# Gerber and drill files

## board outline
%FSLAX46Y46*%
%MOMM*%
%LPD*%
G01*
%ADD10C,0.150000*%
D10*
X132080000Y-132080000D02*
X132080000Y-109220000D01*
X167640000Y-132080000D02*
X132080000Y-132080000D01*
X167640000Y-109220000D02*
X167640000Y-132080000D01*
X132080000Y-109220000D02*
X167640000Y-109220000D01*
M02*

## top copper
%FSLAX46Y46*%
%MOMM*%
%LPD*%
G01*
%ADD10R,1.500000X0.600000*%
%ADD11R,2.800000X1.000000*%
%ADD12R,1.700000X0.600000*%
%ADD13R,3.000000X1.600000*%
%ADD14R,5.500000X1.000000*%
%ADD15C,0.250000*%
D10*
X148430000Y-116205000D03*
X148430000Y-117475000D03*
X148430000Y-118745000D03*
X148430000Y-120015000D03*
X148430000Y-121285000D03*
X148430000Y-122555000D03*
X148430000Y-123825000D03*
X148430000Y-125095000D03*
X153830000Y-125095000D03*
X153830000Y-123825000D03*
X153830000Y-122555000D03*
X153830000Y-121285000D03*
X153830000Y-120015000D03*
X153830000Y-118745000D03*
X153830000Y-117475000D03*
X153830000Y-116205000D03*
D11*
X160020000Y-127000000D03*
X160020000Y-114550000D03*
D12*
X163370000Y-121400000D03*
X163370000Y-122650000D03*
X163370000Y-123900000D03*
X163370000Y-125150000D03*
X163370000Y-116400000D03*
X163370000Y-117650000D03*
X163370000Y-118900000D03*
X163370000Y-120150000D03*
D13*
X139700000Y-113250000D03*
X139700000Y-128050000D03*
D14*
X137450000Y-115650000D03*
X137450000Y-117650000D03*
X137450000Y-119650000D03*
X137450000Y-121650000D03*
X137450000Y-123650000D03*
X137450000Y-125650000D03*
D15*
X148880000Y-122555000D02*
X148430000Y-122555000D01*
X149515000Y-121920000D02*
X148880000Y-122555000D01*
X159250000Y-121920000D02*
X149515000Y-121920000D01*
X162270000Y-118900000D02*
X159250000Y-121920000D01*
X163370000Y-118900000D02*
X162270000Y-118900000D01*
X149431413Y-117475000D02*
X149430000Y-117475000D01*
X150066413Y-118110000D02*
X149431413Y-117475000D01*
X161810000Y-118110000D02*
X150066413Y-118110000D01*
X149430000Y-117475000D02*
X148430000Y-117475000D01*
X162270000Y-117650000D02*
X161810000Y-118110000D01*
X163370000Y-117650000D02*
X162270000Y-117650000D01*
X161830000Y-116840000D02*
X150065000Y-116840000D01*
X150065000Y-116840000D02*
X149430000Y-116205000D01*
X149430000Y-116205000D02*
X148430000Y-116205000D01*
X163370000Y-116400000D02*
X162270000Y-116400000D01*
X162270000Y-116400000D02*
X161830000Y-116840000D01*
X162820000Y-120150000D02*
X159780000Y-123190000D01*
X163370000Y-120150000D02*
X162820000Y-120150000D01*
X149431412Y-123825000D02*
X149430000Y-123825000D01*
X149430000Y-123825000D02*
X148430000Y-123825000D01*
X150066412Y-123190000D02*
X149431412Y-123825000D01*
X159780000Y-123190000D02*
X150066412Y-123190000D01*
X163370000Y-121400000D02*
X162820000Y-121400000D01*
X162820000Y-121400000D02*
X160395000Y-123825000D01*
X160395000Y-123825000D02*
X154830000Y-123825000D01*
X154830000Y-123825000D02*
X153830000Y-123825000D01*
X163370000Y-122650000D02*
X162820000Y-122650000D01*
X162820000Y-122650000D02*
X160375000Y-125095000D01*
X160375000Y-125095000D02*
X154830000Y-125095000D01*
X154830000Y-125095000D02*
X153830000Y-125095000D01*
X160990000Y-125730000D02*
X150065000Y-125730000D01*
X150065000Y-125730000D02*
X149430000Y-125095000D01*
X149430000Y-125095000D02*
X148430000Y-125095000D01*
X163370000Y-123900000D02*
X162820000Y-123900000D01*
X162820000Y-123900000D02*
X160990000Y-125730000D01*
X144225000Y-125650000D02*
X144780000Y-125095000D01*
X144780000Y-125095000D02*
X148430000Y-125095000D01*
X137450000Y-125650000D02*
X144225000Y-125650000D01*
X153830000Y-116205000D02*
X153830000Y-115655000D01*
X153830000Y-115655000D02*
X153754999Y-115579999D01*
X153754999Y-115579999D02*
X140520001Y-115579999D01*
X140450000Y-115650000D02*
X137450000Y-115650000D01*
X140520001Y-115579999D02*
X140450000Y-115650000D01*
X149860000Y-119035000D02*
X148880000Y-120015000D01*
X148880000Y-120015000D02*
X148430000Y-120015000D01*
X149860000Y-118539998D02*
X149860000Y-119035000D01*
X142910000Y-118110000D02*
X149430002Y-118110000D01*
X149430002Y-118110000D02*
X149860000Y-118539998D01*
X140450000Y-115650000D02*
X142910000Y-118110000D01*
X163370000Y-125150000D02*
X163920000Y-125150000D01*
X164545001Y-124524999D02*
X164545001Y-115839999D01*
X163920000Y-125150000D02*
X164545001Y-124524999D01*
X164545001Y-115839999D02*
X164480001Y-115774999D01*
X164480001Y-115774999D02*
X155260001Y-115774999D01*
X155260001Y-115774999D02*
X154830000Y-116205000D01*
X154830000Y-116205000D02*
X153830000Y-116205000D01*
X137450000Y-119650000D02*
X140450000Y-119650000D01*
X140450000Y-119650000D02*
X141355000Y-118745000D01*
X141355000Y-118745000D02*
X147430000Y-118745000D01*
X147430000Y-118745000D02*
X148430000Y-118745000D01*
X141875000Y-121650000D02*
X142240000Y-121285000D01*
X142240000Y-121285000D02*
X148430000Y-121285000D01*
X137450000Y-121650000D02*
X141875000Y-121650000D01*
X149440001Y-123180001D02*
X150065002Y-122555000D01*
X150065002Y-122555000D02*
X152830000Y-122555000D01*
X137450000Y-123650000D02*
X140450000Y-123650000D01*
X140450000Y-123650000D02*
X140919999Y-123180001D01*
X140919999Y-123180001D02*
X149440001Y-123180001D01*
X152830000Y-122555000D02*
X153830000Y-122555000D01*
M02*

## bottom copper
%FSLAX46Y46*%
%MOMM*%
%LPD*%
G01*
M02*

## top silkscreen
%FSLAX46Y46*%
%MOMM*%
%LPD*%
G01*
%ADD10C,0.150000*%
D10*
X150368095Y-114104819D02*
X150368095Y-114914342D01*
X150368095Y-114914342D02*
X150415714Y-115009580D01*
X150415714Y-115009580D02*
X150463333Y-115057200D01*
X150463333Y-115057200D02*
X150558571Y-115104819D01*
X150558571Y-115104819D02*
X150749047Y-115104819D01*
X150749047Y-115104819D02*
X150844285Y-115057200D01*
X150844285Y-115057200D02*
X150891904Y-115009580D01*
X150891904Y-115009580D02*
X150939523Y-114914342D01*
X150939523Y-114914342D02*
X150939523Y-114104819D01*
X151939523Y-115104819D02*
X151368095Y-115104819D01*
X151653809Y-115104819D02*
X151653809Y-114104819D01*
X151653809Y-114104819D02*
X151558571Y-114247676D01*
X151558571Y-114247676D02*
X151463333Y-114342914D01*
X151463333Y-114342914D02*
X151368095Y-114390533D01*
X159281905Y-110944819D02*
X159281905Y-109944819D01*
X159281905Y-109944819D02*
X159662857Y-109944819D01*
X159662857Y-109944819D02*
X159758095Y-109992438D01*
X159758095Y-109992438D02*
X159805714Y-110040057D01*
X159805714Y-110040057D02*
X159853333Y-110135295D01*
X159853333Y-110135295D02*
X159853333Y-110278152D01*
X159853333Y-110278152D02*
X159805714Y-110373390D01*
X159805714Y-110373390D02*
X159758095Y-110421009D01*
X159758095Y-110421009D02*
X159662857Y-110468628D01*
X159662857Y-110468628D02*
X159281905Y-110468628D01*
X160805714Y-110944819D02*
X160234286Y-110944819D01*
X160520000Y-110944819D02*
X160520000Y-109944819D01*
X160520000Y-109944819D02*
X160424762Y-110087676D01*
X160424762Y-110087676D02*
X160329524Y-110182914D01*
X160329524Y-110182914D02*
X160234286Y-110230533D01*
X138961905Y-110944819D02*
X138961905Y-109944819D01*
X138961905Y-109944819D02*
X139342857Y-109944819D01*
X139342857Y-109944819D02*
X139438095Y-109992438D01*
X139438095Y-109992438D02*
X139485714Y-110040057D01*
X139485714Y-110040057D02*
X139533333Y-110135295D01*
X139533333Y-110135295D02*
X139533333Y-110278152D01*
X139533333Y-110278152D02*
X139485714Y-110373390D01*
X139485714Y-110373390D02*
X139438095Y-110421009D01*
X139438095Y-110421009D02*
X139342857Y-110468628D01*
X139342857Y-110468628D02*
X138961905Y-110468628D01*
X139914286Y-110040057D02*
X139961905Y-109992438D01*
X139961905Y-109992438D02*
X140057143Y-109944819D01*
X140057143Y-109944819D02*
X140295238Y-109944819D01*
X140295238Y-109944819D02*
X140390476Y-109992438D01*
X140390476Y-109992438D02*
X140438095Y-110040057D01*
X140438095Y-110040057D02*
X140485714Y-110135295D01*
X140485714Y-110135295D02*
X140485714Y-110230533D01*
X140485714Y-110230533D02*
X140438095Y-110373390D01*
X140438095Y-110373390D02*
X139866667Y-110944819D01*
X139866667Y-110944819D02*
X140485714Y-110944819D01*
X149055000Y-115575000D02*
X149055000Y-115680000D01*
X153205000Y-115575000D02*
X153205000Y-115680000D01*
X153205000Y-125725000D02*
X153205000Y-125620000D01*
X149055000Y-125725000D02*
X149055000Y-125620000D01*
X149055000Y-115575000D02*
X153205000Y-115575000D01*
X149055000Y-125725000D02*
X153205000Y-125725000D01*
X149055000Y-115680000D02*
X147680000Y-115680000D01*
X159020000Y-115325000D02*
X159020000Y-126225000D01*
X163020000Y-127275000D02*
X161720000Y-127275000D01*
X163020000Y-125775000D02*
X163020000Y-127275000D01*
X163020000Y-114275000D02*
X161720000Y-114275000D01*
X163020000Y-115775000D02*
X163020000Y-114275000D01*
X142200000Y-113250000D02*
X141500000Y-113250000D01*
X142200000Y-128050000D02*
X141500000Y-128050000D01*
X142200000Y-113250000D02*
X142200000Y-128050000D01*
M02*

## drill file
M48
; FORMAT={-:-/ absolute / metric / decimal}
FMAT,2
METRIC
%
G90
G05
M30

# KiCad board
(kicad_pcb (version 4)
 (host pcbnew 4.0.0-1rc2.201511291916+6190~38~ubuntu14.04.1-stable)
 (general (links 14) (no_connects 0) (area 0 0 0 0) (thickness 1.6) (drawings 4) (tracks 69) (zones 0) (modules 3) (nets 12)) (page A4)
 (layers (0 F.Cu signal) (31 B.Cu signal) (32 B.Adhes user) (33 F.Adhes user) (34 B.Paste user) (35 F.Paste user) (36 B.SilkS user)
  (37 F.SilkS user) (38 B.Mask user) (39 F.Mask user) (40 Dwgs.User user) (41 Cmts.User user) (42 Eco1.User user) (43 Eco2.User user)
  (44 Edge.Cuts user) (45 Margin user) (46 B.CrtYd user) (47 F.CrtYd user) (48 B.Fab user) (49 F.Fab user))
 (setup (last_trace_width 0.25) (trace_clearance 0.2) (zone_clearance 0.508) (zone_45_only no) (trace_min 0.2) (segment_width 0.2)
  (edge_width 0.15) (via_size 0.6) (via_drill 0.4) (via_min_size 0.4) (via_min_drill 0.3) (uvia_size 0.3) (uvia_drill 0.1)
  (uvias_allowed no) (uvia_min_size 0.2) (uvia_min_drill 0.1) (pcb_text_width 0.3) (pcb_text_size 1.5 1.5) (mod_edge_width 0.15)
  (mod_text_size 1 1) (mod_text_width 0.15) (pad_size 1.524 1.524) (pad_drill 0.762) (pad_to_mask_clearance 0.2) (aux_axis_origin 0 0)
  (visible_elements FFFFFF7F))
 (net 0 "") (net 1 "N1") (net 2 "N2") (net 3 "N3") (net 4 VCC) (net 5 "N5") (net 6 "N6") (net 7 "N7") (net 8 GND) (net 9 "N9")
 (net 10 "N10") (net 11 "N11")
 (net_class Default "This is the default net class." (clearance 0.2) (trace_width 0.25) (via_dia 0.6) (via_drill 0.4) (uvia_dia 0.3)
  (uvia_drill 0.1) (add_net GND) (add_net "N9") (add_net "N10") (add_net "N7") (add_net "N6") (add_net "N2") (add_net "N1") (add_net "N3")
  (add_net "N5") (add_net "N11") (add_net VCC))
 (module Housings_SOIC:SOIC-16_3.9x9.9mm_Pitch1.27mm (layer F.Cu) (at 151.13 120.65)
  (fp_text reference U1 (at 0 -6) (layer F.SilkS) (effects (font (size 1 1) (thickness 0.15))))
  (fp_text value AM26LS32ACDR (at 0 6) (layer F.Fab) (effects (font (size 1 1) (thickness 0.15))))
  (fp_line (start -2.075 -5.075) (end -2.075 -4.97) (layer F.SilkS) (width 0.15))
  (fp_line (start 2.075 -5.075) (end 2.075 -4.97) (layer F.SilkS) (width 0.15))
  (fp_line (start 2.075 5.075) (end 2.075 4.97) (layer F.SilkS) (width 0.15))
  (fp_line (start -2.075 5.075) (end -2.075 4.97) (layer F.SilkS) (width 0.15))
  (fp_line (start -2.075 -5.075) (end 2.075 -5.075) (layer F.SilkS) (width 0.15))
  (fp_line (start -2.075 5.075) (end 2.075 5.075) (layer F.SilkS) (width 0.15))
  (fp_line (start -2.075 -4.97) (end -3.45 -4.97) (layer F.SilkS) (width 0.15))
  (pad 1 smd rect (at -2.7 -4.445) (size 1.5 0.6) (layers F.Cu F.Paste F.Mask) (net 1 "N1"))
  (pad 2 smd rect (at -2.7 -3.175) (size 1.5 0.6) (layers F.Cu F.Paste F.Mask) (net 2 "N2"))
  (pad 3 smd rect (at -2.7 -1.905) (size 1.5 0.6) (layers F.Cu F.Paste F.Mask) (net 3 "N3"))
  (pad 4 smd rect (at -2.7 -0.635) (size 1.5 0.6) (layers F.Cu F.Paste F.Mask) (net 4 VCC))
  (pad 5 smd rect (at -2.7 0.635) (size 1.5 0.6) (layers F.Cu F.Paste F.Mask) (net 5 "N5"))
  (pad 6 smd rect (at -2.7 1.905) (size 1.5 0.6) (layers F.Cu F.Paste F.Mask) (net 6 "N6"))
  (pad 7 smd rect (at -2.7 3.175) (size 1.5 0.6) (layers F.Cu F.Paste F.Mask) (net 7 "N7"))
  (pad 8 smd rect (at -2.7 4.445) (size 1.5 0.6) (layers F.Cu F.Paste F.Mask) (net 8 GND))
  (pad 9 smd rect (at 2.7 4.445) (size 1.5 0.6) (layers F.Cu F.Paste F.Mask) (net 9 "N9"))
  (pad 10 smd rect (at 2.7 3.175) (size 1.5 0.6) (layers F.Cu F.Paste F.Mask) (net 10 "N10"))
  (pad 11 smd rect (at 2.7 1.905) (size 1.5 0.6) (layers F.Cu F.Paste F.Mask) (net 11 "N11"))
  (pad 12 smd rect (at 2.7 0.635) (size 1.5 0.6) (layers F.Cu F.Paste F.Mask))
  (pad 13 smd rect (at 2.7 -0.635) (size 1.5 0.6) (layers F.Cu F.Paste F.Mask))
  (pad 14 smd rect (at 2.7 -1.905) (size 1.5 0.6) (layers F.Cu F.Paste F.Mask))
  (pad 15 smd rect (at 2.7 -3.175) (size 1.5 0.6) (layers F.Cu F.Paste F.Mask))
  (pad 16 smd rect (at 2.7 -4.445) (size 1.5 0.6) (layers F.Cu F.Paste F.Mask) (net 4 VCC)))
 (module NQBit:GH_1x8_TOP (layer F.Cu) (at 160.02 120.775 270)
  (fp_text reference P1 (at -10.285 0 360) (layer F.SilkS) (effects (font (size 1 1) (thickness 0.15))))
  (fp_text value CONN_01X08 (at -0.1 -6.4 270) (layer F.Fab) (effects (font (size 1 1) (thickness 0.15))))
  (fp_line (start -5.45 1) (end 5.45 1) (layer F.SilkS) (width 0.15))
  (fp_line (start 6.5 -3) (end 6.5 -1.7) (layer F.SilkS) (width 0.15))
  (fp_line (start 5 -3) (end 6.5 -3) (layer F.SilkS) (width 0.15))
  (fp_line (start -6.5 -3) (end -6.5 -1.7) (layer F.SilkS) (width 0.15))
  (fp_line (start -5 -3) (end -6.5 -3) (layer F.SilkS) (width 0.15))
  (pad MECH smd rect (at 6.225 0 270) (size 1 2.8) (layers F.Cu F.Paste F.Mask))
  (pad MECH smd rect (at -6.225 0 270) (size 1 2.8) (layers F.Cu F.Paste F.Mask))
  (pad 4 smd rect (at 0.625 -3.35 270) (size 0.6 1.7) (layers F.Cu F.Paste F.Mask) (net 10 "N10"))
  (pad 3 smd rect (at 1.875 -3.35 270) (size 0.6 1.7) (layers F.Cu F.Paste F.Mask) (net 9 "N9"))
  (pad 2 smd rect (at 3.125 -3.35 270) (size 0.6 1.7) (layers F.Cu F.Paste F.Mask) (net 8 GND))
  (pad 1 smd rect (at 4.375 -3.35 270) (size 0.6 1.7) (layers F.Cu F.Paste F.Mask) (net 4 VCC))
  (pad 8 smd rect (at -4.375 -3.35 270) (size 0.6 1.7) (layers F.Cu F.Paste F.Mask) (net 1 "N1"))
  (pad 7 smd rect (at -3.125 -3.35 270) (size 0.6 1.7) (layers F.Cu F.Paste F.Mask) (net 2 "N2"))
  (pad 6 smd rect (at -1.875 -3.35 270) (size 0.6 1.7) (layers F.Cu F.Paste F.Mask) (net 6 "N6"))
  (pad 5 smd rect (at -0.625 -3.35 270) (size 0.6 1.7) (layers F.Cu F.Paste F.Mask) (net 7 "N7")))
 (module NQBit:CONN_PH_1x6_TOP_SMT (layer F.Cu) (at 139.7 120.65 270)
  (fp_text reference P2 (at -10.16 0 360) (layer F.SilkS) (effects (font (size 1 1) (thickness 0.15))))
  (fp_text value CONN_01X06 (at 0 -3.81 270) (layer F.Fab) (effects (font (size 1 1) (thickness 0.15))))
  (fp_line (start -7.4 -2.5) (end -7.4 -1.8) (layer F.SilkS) (width 0.15))
  (fp_line (start 7.4 -2.5) (end 7.4 -1.8) (layer F.SilkS) (width 0.15))
  (fp_line (start -7.4 -2.5) (end 7.4 -2.5) (layer F.SilkS) (width 0.15))
  (pad MECH smd rect (at -7.4 0 270) (size 1.6 3) (layers F.Cu F.Paste F.Mask))
  (pad MECH smd rect (at 7.4 0 270) (size 1.6 3) (layers F.Cu F.Paste F.Mask))
  (pad 1 smd rect (at -5 2.25 270) (size 1 5.5) (layers F.Cu F.Paste F.Mask) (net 4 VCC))
  (pad 2 smd rect (at -3 2.25 270) (size 1 5.5) (layers F.Cu F.Paste F.Mask))
  (pad 3 smd rect (at -1 2.25 270) (size 1 5.5) (layers F.Cu F.Paste F.Mask) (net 3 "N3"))
  (pad 4 smd rect (at 1 2.25 270) (size 1 5.5) (layers F.Cu F.Paste F.Mask) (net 5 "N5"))
  (pad 5 smd rect (at 3 2.25 270) (size 1 5.5) (layers F.Cu F.Paste F.Mask) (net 11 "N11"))
  (pad 6 smd rect (at 5 2.25 270) (size 1 5.5) (layers F.Cu F.Paste F.Mask) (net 8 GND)))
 (gr_line (start 132.08 132.08) (end 132.08 109.22) (layer Edge.Cuts) (width 0.15))
 (gr_line (start 167.64 132.08) (end 132.08 132.08) (layer Edge.Cuts) (width 0.15))
 (gr_line (start 167.64 109.22) (end 167.64 132.08) (layer Edge.Cuts) (width 0.15))
 (gr_line (start 132.08 109.22) (end 167.64 109.22) (layer Edge.Cuts) (width 0.15))
 (segment (start 148.88 122.555) (end 148.43 122.555) (width 0.25) (layer F.Cu) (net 6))
 (segment (start 149.515 121.92) (end 148.88 122.555) (width 0.25) (layer F.Cu) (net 6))
 (segment (start 159.25 121.92) (end 149.515 121.92) (width 0.25) (layer F.Cu) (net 6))
 (segment (start 162.27 118.9) (end 159.25 121.92) (width 0.25) (layer F.Cu) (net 6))
 (segment (start 163.37 118.9) (end 162.27 118.9) (width 0.25) (layer F.Cu) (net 6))
 (segment (start 149.431413 117.475) (end 149.43 117.475) (width 0.25) (layer F.Cu) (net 2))
 (segment (start 150.066413 118.11) (end 149.431413 117.475) (width 0.25) (layer F.Cu) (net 2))
 (segment (start 161.81 118.11) (end 150.066413 118.11) (width 0.25) (layer F.Cu) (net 2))
 (segment (start 149.43 117.475) (end 148.43 117.475) (width 0.25) (layer F.Cu) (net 2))
 (segment (start 162.27 117.65) (end 161.81 118.11) (width 0.25) (layer F.Cu) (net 2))
 (segment (start 163.37 117.65) (end 162.27 117.65) (width 0.25) (layer F.Cu) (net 2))
 (segment (start 161.83 116.84) (end 150.065 116.84) (width 0.25) (layer F.Cu) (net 1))
 (segment (start 150.065 116.84) (end 149.43 116.205) (width 0.25) (layer F.Cu) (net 1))
 (segment (start 149.43 116.205) (end 148.43 116.205) (width 0.25) (layer F.Cu) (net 1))
 (segment (start 163.37 116.4) (end 162.27 116.4) (width 0.25) (layer F.Cu) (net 1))
 (segment (start 162.27 116.4) (end 161.83 116.84) (width 0.25) (layer F.Cu) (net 1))
 (segment (start 162.82 120.15) (end 159.78 123.19) (width 0.25) (layer F.Cu) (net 7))
 (segment (start 163.37 120.15) (end 162.82 120.15) (width 0.25) (layer F.Cu) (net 7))
 (segment (start 149.431412 123.825) (end 149.43 123.825) (width 0.25) (layer F.Cu) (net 7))
 (segment (start 149.43 123.825) (end 148.43 123.825) (width 0.25) (layer F.Cu) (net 7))
 (segment (start 150.066412 123.19) (end 149.431412 123.825) (width 0.25) (layer F.Cu) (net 7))
 (segment (start 159.78 123.19) (end 150.066412 123.19) (width 0.25) (layer F.Cu) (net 7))
 (segment (start 163.37 121.4) (end 162.82 121.4) (width 0.25) (layer F.Cu) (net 10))
 (segment (start 162.82 121.4) (end 160.395 123.825) (width 0.25) (layer F.Cu) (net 10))
 (segment (start 160.395 123.825) (end 154.83 123.825) (width 0.25) (layer F.Cu) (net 10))
 (segment (start 154.83 123.825) (end 153.83 123.825) (width 0.25) (layer F.Cu) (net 10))
 (segment (start 163.37 122.65) (end 162.82 122.65) (width 0.25) (layer F.Cu) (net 9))
 (segment (start 162.82 122.65) (end 160.375 125.095) (width 0.25) (layer F.Cu) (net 9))
 (segment (start 160.375 125.095) (end 154.83 125.095) (width 0.25) (layer F.Cu) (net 9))
 (segment (start 154.83 125.095) (end 153.83 125.095) (width 0.25) (layer F.Cu) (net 9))
 (segment (start 160.99 125.73) (end 150.065 125.73) (width 0.25) (layer F.Cu) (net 8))
 (segment (start 150.065 125.73) (end 149.43 125.095) (width 0.25) (layer F.Cu) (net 8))
 (segment (start 149.43 125.095) (end 148.43 125.095) (width 0.25) (layer F.Cu) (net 8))
 (segment (start 163.37 123.9) (end 162.82 123.9) (width 0.25) (layer F.Cu) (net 8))
 (segment (start 162.82 123.9) (end 160.99 125.73) (width 0.25) (layer F.Cu) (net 8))
 (segment (start 144.225 125.65) (end 144.78 125.095) (width 0.25) (layer F.Cu) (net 8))
 (segment (start 144.78 125.095) (end 148.43 125.095) (width 0.25) (layer F.Cu) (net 8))
 (segment (start 137.45 125.65) (end 144.225 125.65) (width 0.25) (layer F.Cu) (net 8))
 (segment (start 153.83 116.205) (end 153.83 115.655) (width 0.25) (layer F.Cu) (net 4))
 (segment (start 153.83 115.655) (end 153.754999 115.579999) (width 0.25) (layer F.Cu) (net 4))
 (segment (start 153.754999 115.579999) (end 140.520001 115.579999) (width 0.25) (layer F.Cu) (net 4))
 (segment (start 140.45 115.65) (end 137.45 115.65) (width 0.25) (layer F.Cu) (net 4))
 (segment (start 140.520001 115.579999) (end 140.45 115.65) (width 0.25) (layer F.Cu) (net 4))
 (segment (start 149.86 119.035) (end 148.88 120.015) (width 0.25) (layer F.Cu) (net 4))
 (segment (start 148.88 120.015) (end 148.43 120.015) (width 0.25) (layer F.Cu) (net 4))
 (segment (start 149.86 118.539998) (end 149.86 119.035) (width 0.25) (layer F.Cu) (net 4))
 (segment (start 142.91 118.11) (end 149.430002 118.11) (width 0.25) (layer F.Cu) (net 4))
 (segment (start 149.430002 118.11) (end 149.86 118.539998) (width 0.25) (layer F.Cu) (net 4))
 (segment (start 140.45 115.65) (end 142.91 118.11) (width 0.25) (layer F.Cu) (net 4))
 (segment (start 163.37 125.15) (end 163.92 125.15) (width 0.25) (layer F.Cu) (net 4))
 (segment (start 164.545001 124.524999) (end 164.545001 115.839999) (width 0.25) (layer F.Cu) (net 4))
 (segment (start 163.92 125.15) (end 164.545001 124.524999) (width 0.25) (layer F.Cu) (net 4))
 (segment (start 164.545001 115.839999) (end 164.480001 115.774999) (width 0.25) (layer F.Cu) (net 4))
 (segment (start 164.480001 115.774999) (end 155.260001 115.774999) (width 0.25) (layer F.Cu) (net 4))
 (segment (start 155.260001 115.774999) (end 154.83 116.205) (width 0.25) (layer F.Cu) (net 4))
 (segment (start 154.83 116.205) (end 153.83 116.205) (width 0.25) (layer F.Cu) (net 4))
 (segment (start 137.45 119.65) (end 140.45 119.65) (width 0.25) (layer F.Cu) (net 3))
 (segment (start 140.45 119.65) (end 141.355 118.745) (width 0.25) (layer F.Cu) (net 3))
 (segment (start 141.355 118.745) (end 147.43 118.745) (width 0.25) (layer F.Cu) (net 3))
 (segment (start 147.43 118.745) (end 148.43 118.745) (width 0.25) (layer F.Cu) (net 3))
 (segment (start 141.875 121.65) (end 142.24 121.285) (width 0.25) (layer F.Cu) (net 5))
 (segment (start 142.24 121.285) (end 148.43 121.285) (width 0.25) (layer F.Cu) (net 5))
 (segment (start 137.45 121.65) (end 141.875 121.65) (width 0.25) (layer F.Cu) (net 5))
 (segment (start 149.440001 123.180001) (end 150.065002 122.555) (width 0.25) (layer F.Cu) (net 11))
 (segment (start 150.065002 122.555) (end 152.83 122.555) (width 0.25) (layer F.Cu) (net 11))
 (segment (start 137.45 123.65) (end 140.45 123.65) (width 0.25) (layer F.Cu) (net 11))
 (segment (start 140.45 123.65) (end 140.919999 123.180001) (width 0.25) (layer F.Cu) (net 11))
 (segment (start 140.919999 123.180001) (end 149.440001 123.180001) (width 0.25) (layer F.Cu) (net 11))
 (segment (start 152.83 122.555) (end 153.83 122.555) (width 0.25) (layer F.Cu) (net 11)))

